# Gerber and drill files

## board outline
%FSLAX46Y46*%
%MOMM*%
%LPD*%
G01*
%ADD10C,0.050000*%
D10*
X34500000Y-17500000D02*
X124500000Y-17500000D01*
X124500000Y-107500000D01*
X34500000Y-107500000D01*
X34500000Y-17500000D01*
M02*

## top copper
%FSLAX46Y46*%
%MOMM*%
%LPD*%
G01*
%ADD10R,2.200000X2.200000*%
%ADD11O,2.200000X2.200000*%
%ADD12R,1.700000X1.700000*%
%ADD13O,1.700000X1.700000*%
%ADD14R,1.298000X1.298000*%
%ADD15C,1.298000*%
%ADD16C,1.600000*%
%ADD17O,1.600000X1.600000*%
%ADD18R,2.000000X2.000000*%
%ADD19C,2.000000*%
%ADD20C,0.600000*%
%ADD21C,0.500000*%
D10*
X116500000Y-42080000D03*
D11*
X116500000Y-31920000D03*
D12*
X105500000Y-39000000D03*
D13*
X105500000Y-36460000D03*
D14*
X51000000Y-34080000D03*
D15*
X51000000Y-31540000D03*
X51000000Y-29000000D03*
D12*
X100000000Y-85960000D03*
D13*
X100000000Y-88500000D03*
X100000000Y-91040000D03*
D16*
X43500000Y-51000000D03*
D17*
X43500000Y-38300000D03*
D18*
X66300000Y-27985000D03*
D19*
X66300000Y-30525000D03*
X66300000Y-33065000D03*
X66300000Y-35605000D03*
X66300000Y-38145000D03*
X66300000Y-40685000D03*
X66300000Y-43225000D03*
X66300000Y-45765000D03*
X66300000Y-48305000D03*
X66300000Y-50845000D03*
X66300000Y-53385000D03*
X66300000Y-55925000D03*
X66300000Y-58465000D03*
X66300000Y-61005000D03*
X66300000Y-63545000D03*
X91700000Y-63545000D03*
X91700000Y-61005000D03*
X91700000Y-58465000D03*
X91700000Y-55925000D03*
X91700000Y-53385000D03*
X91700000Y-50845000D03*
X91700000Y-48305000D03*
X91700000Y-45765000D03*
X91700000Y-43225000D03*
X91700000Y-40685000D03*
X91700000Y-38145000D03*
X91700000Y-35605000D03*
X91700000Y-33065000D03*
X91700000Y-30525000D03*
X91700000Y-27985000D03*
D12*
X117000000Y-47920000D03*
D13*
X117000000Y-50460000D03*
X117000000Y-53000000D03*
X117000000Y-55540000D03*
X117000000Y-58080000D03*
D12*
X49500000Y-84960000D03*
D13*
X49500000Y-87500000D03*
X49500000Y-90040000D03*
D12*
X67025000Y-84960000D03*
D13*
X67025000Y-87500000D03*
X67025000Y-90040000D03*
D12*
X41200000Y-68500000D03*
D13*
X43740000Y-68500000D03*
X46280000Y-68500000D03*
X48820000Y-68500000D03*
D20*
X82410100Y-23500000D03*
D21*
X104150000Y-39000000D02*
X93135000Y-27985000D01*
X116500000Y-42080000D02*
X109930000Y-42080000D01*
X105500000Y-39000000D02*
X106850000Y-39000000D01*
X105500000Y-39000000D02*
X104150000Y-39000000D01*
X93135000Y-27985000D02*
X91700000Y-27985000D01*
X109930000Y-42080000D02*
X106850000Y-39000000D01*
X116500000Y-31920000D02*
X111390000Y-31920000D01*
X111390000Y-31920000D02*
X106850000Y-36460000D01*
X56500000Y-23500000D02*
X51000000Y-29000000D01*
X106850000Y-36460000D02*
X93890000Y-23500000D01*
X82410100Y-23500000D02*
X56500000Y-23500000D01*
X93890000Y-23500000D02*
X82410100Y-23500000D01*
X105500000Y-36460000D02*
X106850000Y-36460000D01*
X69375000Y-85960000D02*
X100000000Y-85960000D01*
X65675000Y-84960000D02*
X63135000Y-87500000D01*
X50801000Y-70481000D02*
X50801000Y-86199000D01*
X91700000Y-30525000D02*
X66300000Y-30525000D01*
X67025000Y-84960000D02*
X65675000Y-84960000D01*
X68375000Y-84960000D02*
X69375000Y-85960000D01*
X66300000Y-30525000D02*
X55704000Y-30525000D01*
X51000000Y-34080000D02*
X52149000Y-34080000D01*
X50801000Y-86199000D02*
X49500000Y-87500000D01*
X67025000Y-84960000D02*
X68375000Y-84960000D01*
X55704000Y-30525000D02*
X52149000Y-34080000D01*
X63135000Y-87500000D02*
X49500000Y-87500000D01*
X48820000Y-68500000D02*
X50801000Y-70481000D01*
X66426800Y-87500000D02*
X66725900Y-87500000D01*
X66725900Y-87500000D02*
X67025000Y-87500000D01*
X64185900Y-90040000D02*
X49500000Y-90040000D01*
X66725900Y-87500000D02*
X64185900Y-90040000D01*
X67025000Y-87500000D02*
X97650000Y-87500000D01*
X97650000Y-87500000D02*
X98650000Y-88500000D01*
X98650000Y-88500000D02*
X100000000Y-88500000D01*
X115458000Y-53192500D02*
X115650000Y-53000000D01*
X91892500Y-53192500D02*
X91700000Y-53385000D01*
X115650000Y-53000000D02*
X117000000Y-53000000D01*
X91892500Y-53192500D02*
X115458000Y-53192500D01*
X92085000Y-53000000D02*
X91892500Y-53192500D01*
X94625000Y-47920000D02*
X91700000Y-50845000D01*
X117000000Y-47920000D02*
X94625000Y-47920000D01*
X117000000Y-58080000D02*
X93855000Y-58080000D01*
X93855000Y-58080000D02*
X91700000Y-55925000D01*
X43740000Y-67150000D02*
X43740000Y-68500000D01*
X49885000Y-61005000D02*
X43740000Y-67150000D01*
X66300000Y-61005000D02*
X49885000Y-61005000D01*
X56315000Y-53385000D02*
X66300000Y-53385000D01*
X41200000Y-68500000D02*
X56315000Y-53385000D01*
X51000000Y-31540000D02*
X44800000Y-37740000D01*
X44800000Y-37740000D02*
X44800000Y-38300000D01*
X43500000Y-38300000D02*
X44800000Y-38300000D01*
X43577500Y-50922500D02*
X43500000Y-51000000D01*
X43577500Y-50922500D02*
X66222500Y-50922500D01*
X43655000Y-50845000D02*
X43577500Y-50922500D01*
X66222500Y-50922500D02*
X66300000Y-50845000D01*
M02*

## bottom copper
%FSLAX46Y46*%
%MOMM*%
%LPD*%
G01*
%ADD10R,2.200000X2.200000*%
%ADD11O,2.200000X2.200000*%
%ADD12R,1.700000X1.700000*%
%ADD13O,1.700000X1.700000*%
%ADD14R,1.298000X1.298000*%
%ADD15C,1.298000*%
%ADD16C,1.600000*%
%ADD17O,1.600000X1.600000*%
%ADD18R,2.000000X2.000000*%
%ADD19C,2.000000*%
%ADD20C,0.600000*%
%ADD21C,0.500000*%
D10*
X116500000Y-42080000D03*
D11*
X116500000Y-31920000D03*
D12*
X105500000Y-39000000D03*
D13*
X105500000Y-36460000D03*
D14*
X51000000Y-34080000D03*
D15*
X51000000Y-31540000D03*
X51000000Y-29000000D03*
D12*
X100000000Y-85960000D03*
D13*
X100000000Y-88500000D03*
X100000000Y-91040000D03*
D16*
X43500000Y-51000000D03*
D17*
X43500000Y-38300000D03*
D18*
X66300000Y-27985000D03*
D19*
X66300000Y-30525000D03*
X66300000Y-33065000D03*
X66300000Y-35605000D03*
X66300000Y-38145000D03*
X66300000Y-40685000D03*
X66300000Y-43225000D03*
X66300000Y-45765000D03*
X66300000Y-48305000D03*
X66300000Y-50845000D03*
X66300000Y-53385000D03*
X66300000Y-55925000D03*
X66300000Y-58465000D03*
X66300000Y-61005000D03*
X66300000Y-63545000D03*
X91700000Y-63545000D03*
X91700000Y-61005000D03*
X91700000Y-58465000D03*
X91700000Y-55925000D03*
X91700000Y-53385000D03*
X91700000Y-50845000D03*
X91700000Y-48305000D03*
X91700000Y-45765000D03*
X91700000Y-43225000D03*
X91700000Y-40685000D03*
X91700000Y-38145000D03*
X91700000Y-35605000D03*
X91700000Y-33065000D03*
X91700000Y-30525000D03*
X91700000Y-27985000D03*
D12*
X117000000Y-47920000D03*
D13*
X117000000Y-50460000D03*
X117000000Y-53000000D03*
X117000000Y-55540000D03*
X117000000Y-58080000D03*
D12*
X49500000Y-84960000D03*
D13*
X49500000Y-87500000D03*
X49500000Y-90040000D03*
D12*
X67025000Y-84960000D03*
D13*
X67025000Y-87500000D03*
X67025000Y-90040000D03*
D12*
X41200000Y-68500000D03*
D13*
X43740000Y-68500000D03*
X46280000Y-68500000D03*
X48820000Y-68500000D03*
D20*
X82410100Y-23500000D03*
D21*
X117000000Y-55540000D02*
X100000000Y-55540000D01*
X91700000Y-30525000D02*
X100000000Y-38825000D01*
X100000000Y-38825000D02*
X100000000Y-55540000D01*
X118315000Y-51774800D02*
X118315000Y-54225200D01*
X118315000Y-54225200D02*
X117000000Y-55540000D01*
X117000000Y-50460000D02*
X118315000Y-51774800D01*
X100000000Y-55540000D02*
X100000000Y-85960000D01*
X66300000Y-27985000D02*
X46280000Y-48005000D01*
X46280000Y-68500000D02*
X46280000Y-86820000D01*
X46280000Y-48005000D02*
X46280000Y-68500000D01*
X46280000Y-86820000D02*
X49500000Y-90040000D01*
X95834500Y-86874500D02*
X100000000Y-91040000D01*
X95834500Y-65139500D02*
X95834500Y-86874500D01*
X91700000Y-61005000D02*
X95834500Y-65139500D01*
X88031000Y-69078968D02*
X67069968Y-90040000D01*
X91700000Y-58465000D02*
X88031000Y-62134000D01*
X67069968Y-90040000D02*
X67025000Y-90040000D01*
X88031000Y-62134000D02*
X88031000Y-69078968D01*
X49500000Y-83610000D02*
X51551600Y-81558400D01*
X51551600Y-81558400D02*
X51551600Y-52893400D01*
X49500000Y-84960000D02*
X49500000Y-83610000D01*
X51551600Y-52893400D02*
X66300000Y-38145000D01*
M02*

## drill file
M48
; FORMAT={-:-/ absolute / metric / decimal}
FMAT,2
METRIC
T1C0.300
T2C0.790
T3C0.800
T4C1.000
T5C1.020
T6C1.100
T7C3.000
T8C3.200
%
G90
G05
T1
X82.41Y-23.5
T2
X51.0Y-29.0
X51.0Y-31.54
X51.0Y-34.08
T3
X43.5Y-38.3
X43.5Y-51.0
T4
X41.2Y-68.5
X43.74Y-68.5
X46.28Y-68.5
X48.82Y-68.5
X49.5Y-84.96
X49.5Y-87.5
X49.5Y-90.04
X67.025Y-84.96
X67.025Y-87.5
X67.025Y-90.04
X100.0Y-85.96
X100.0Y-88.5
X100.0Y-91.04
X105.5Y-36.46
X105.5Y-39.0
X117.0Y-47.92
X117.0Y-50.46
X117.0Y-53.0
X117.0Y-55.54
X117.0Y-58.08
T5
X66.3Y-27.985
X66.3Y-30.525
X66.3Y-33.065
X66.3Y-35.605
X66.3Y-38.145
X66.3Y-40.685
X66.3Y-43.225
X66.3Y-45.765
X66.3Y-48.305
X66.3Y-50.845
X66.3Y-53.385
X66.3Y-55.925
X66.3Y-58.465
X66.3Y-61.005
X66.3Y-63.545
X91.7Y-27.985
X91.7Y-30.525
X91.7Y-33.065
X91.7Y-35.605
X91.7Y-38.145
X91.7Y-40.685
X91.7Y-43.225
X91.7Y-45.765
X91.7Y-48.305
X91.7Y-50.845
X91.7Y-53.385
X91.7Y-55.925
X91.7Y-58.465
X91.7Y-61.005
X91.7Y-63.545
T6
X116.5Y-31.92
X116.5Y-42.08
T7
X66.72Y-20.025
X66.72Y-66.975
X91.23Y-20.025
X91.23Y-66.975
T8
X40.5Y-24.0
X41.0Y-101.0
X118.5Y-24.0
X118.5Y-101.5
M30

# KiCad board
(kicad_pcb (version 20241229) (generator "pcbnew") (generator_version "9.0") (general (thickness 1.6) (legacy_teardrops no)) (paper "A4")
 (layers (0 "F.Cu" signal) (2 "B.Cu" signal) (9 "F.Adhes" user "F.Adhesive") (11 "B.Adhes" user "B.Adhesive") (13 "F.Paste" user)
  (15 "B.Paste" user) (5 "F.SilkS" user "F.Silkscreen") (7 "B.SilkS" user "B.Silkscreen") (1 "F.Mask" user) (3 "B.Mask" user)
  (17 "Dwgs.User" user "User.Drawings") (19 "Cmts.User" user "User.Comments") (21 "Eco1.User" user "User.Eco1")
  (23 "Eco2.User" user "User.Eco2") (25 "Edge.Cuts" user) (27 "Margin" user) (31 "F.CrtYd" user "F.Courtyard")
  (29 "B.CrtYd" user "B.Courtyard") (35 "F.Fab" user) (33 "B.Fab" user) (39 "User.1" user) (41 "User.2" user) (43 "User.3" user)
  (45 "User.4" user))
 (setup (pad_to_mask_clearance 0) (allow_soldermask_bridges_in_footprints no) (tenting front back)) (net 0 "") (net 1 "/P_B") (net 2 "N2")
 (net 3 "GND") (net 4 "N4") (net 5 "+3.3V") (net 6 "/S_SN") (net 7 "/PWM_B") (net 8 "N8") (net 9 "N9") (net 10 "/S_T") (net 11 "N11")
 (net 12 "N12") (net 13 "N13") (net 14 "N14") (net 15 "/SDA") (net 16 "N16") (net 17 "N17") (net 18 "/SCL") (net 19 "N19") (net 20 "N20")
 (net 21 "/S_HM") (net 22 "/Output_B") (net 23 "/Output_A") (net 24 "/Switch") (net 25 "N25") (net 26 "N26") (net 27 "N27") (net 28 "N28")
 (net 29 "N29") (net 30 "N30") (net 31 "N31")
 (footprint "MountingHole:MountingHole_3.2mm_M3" (layer "F.Cu") (at 118.5 101.5)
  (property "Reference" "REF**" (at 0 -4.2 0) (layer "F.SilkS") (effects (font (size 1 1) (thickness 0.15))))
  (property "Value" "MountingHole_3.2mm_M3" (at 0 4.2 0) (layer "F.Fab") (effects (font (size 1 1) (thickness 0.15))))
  (pad "" np_thru_hole circle (at 0 0) (size 3.2 3.2) (drill 3.2) (layers "*.Cu" "*.Mask")))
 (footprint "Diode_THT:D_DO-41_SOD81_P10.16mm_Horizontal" (layer "F.Cu") (at 116.5 42.08 90)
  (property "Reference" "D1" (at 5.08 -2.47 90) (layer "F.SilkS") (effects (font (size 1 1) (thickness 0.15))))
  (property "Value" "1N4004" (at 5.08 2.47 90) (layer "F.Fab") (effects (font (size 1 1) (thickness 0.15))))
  (pad "1" thru_hole rect (at 0 0 90) (size 2.2 2.2) (drill 1.1) (layers "*.Cu" "*.Mask") (remove_unused_layers no) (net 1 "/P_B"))
  (pad "2" thru_hole oval (at 10.16 0 90) (size 2.2 2.2) (drill 1.1) (layers "*.Cu" "*.Mask") (remove_unused_layers no) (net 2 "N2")))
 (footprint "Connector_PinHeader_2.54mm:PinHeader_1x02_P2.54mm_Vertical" (layer "F.Cu") (at 105.5 39 180)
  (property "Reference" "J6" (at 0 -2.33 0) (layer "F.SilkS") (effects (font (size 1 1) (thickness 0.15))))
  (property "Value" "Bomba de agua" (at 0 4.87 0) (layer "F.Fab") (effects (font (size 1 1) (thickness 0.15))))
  (pad "1" thru_hole rect (at 0 0 180) (size 1.7 1.7) (drill 1) (layers "*.Cu" "*.Mask") (remove_unused_layers no) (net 1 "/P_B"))
  (pad "2" thru_hole oval (at 0 2.54 180) (size 1.7 1.7) (drill 1) (layers "*.Cu" "*.Mask") (remove_unused_layers no) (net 2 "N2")))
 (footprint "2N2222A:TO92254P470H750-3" (layer "F.Cu") (at 48.67 31.54 90)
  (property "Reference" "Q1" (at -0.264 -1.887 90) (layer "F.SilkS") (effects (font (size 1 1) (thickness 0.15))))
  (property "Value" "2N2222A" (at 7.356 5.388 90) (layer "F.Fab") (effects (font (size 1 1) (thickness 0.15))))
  (pad "1" thru_hole rect (at -2.54 2.33 90) (size 1.298 1.298) (drill 0.79) (layers "*.Cu" "*.Mask") (remove_unused_layers no)
   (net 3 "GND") (solder_mask_margin 0.102))
  (pad "2" thru_hole circle (at 0 2.33 90) (size 1.298 1.298) (drill 0.79) (layers "*.Cu" "*.Mask") (remove_unused_layers no) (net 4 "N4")
   (solder_mask_margin 0.102))
  (pad "3" thru_hole circle (at 2.54 2.33 90) (size 1.298 1.298) (drill 0.79) (layers "*.Cu" "*.Mask") (remove_unused_layers no)
   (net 2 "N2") (solder_mask_margin 0.102)))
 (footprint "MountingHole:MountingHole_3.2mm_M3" (layer "F.Cu") (at 41 101)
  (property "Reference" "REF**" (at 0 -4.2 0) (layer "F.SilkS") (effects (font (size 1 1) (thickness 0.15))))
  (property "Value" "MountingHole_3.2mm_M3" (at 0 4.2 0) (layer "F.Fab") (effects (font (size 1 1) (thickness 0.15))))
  (pad "" np_thru_hole circle (at 0 0) (size 3.2 3.2) (drill 3.2) (layers "*.Cu" "*.Mask")))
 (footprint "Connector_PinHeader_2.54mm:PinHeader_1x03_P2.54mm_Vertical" (layer "F.Cu") (at 100 85.96)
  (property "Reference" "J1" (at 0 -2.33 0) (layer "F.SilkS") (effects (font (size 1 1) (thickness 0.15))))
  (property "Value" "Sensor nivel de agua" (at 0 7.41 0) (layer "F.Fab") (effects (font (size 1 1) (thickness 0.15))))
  (pad "1" thru_hole rect (at 0 0) (size 1.7 1.7) (drill 1) (layers "*.Cu" "*.Mask") (remove_unused_layers no) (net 3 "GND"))
  (pad "2" thru_hole oval (at 0 2.54) (size 1.7 1.7) (drill 1) (layers "*.Cu" "*.Mask") (remove_unused_layers no) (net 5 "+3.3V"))
  (pad "3" thru_hole oval (at 0 5.08) (size 1.7 1.7) (drill 1) (layers "*.Cu" "*.Mask") (remove_unused_layers no) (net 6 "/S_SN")))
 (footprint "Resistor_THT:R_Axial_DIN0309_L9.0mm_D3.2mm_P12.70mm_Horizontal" (layer "F.Cu") (at 43.5 51 90)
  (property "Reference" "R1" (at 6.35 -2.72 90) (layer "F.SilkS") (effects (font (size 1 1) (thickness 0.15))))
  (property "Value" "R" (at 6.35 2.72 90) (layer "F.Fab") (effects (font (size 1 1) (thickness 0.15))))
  (pad "1" thru_hole circle (at 0 0 90) (size 1.6 1.6) (drill 0.8) (layers "*.Cu" "*.Mask") (remove_unused_layers no) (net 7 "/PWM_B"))
  (pad "2" thru_hole oval (at 12.7 0 90) (size 1.6 1.6) (drill 0.8) (layers "*.Cu" "*.Mask") (remove_unused_layers no) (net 4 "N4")))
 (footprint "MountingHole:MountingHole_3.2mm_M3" (layer "F.Cu") (at 118.5 24)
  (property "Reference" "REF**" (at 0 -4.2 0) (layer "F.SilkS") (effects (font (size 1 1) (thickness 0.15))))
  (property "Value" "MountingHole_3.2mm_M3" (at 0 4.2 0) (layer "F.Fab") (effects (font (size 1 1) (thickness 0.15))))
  (pad "" np_thru_hole circle (at 0 0) (size 3.2 3.2) (drill 3.2) (layers "*.Cu" "*.Mask")))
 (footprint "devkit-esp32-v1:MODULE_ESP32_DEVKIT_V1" (layer "F.Cu") (at 79 43.5)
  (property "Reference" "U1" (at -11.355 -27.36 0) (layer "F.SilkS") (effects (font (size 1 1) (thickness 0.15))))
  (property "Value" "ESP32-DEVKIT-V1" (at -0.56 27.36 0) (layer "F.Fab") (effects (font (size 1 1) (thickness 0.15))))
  (pad "" np_thru_hole circle (at -12.28 -23.475) (size 3 3) (drill 3) (layers "*.Cu" "*.Mask"))
  (pad "" np_thru_hole circle (at -12.28 23.475) (size 3 3) (drill 3) (layers "*.Cu" "*.Mask"))
  (pad "" np_thru_hole circle (at 12.23 -23.475) (size 3 3) (drill 3) (layers "*.Cu" "*.Mask"))
  (pad "" np_thru_hole circle (at 12.23 23.475) (size 3 3) (drill 3) (layers "*.Cu" "*.Mask"))
  (pad "1" thru_hole rect (at -12.7 -15.515) (size 2 2) (drill 1.02) (layers "*.Cu" "*.Mask") (remove_unused_layers no) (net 5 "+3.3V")
   (solder_mask_margin 0.102))
  (pad "2" thru_hole circle (at -12.7 -12.975) (size 2 2) (drill 1.02) (layers "*.Cu" "*.Mask") (remove_unused_layers no) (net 3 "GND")
   (solder_mask_margin 0.102))
  (pad "3" thru_hole circle (at -12.7 -10.435) (size 2 2) (drill 1.02) (layers "*.Cu" "*.Mask") (remove_unused_layers no) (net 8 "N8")
   (solder_mask_margin 0.102))
  (pad "4" thru_hole circle (at -12.7 -7.895) (size 2 2) (drill 1.02) (layers "*.Cu" "*.Mask") (remove_unused_layers no) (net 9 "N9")
   (solder_mask_margin 0.102))
  (pad "5" thru_hole circle (at -12.7 -5.355) (size 2 2) (drill 1.02) (layers "*.Cu" "*.Mask") (remove_unused_layers no) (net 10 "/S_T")
   (solder_mask_margin 0.102))
  (pad "6" thru_hole circle (at -12.7 -2.815) (size 2 2) (drill 1.02) (layers "*.Cu" "*.Mask") (remove_unused_layers no) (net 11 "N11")
   (solder_mask_margin 0.102))
  (pad "7" thru_hole circle (at -12.7 -0.275) (size 2 2) (drill 1.02) (layers "*.Cu" "*.Mask") (remove_unused_layers no) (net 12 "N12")
   (solder_mask_margin 0.102))
  (pad "8" thru_hole circle (at -12.7 2.265) (size 2 2) (drill 1.02) (layers "*.Cu" "*.Mask") (remove_unused_layers no) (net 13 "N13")
   (solder_mask_margin 0.102))
  (pad "9" thru_hole circle (at -12.7 4.805) (size 2 2) (drill 1.02) (layers "*.Cu" "*.Mask") (remove_unused_layers no) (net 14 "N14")
   (solder_mask_margin 0.102))
  (pad "10" thru_hole circle (at -12.7 7.345) (size 2 2) (drill 1.02) (layers "*.Cu" "*.Mask") (remove_unused_layers no) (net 7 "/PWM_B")
   (solder_mask_margin 0.102))
  (pad "11" thru_hole circle (at -12.7 9.885) (size 2 2) (drill 1.02) (layers "*.Cu" "*.Mask") (remove_unused_layers no) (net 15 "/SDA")
   (solder_mask_margin 0.102))
  (pad "12" thru_hole circle (at -12.7 12.425) (size 2 2) (drill 1.02) (layers "*.Cu" "*.Mask") (remove_unused_layers no) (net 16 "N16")
   (solder_mask_margin 0.102))
  (pad "13" thru_hole circle (at -12.7 14.965) (size 2 2) (drill 1.02) (layers "*.Cu" "*.Mask") (remove_unused_layers no) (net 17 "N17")
   (solder_mask_margin 0.102))
  (pad "14" thru_hole circle (at -12.7 17.505) (size 2 2) (drill 1.02) (layers "*.Cu" "*.Mask") (remove_unused_layers no) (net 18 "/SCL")
   (solder_mask_margin 0.102))
  (pad "15" thru_hole circle (at -12.7 20.045) (size 2 2) (drill 1.02) (layers "*.Cu" "*.Mask") (remove_unused_layers no) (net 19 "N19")
   (solder_mask_margin 0.102))
  (pad "16" thru_hole circle (at 12.7 20.045) (size 2 2) (drill 1.02) (layers "*.Cu" "*.Mask") (remove_unused_layers no) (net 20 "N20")
   (solder_mask_margin 0.102))
  (pad "17" thru_hole circle (at 12.7 17.505) (size 2 2) (drill 1.02) (layers "*.Cu" "*.Mask") (remove_unused_layers no) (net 6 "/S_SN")
   (solder_mask_margin 0.102))
  (pad "18" thru_hole circle (at 12.7 14.965) (size 2 2) (drill 1.02) (layers "*.Cu" "*.Mask") (remove_unused_layers no) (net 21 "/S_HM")
   (solder_mask_margin 0.102))
  (pad "19" thru_hole circle (at 12.7 12.425) (size 2 2) (drill 1.02) (layers "*.Cu" "*.Mask") (remove_unused_layers no)
   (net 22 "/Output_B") (solder_mask_margin 0.102))
  (pad "20" thru_hole circle (at 12.7 9.885) (size 2 2) (drill 1.02) (layers "*.Cu" "*.Mask") (remove_unused_layers no) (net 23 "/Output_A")
   (solder_mask_margin 0.102))
  (pad "21" thru_hole circle (at 12.7 7.345) (size 2 2) (drill 1.02) (layers "*.Cu" "*.Mask") (remove_unused_layers no) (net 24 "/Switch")
   (solder_mask_margin 0.102))
  (pad "22" thru_hole circle (at 12.7 4.805) (size 2 2) (drill 1.02) (layers "*.Cu" "*.Mask") (remove_unused_layers no) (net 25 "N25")
   (solder_mask_margin 0.102))
  (pad "23" thru_hole circle (at 12.7 2.265) (size 2 2) (drill 1.02) (layers "*.Cu" "*.Mask") (remove_unused_layers no) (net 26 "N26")
   (solder_mask_margin 0.102))
  (pad "24" thru_hole circle (at 12.7 -0.275) (size 2 2) (drill 1.02) (layers "*.Cu" "*.Mask") (remove_unused_layers no) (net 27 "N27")
   (solder_mask_margin 0.102))
  (pad "25" thru_hole circle (at 12.7 -2.815) (size 2 2) (drill 1.02) (layers "*.Cu" "*.Mask") (remove_unused_layers no) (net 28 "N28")
   (solder_mask_margin 0.102))
  (pad "26" thru_hole circle (at 12.7 -5.355) (size 2 2) (drill 1.02) (layers "*.Cu" "*.Mask") (remove_unused_layers no) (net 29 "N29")
   (solder_mask_margin 0.102))
  (pad "27" thru_hole circle (at 12.7 -7.895) (size 2 2) (drill 1.02) (layers "*.Cu" "*.Mask") (remove_unused_layers no) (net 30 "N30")
   (solder_mask_margin 0.102))
  (pad "28" thru_hole circle (at 12.7 -10.435) (size 2 2) (drill 1.02) (layers "*.Cu" "*.Mask") (remove_unused_layers no) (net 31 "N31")
   (solder_mask_margin 0.102))
  (pad "29" thru_hole circle (at 12.7 -12.975) (size 2 2) (drill 1.02) (layers "*.Cu" "*.Mask") (remove_unused_layers no) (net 3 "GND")
   (solder_mask_margin 0.102))
  (pad "30" thru_hole circle (at 12.7 -15.515) (size 2 2) (drill 1.02) (layers "*.Cu" "*.Mask") (remove_unused_layers no) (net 1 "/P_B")
   (solder_mask_margin 0.102))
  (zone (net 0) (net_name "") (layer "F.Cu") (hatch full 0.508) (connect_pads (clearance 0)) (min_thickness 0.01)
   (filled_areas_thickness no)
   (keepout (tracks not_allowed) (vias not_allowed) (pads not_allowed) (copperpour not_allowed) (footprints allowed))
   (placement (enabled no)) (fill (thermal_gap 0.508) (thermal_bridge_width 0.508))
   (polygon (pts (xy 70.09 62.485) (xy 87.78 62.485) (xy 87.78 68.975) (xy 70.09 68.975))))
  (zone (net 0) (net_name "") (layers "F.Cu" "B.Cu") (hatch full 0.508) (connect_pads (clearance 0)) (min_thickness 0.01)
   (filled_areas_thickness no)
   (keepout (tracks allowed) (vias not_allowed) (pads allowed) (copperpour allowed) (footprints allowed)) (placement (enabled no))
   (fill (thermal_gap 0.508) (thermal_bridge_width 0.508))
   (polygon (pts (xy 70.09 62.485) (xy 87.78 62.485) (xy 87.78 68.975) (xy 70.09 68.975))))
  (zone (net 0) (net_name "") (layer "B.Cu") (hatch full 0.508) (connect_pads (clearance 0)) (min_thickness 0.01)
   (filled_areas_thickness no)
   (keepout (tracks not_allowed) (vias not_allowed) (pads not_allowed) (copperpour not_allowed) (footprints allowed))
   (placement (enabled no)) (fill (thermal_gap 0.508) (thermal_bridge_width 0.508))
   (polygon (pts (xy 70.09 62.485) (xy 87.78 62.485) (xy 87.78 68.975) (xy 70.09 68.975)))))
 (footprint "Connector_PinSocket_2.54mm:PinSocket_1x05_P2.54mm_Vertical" (layer "F.Cu") (at 117 47.92)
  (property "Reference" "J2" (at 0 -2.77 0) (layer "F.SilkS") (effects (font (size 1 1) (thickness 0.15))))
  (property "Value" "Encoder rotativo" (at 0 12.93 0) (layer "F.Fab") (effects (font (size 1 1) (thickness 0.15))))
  (pad "1" thru_hole rect (at 0 0) (size 1.7 1.7) (drill 1) (layers "*.Cu" "*.Mask") (remove_unused_layers no) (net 24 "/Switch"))
  (pad "2" thru_hole oval (at 0 2.54) (size 1.7 1.7) (drill 1) (layers "*.Cu" "*.Mask") (remove_unused_layers no) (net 3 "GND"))
  (pad "3" thru_hole oval (at 0 5.08) (size 1.7 1.7) (drill 1) (layers "*.Cu" "*.Mask") (remove_unused_layers no) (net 23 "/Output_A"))
  (pad "4" thru_hole oval (at 0 7.62) (size 1.7 1.7) (drill 1) (layers "*.Cu" "*.Mask") (remove_unused_layers no) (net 3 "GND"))
  (pad "5" thru_hole oval (at 0 10.16) (size 1.7 1.7) (drill 1) (layers "*.Cu" "*.Mask") (remove_unused_layers no) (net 22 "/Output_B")))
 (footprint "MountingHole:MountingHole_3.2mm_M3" (layer "F.Cu") (at 40.5 24)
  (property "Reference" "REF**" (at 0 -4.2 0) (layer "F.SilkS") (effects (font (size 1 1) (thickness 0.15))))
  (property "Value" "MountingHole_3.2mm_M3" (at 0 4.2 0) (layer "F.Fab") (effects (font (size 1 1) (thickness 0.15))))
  (pad "" np_thru_hole circle (at 0 0) (size 3.2 3.2) (drill 3.2) (layers "*.Cu" "*.Mask")))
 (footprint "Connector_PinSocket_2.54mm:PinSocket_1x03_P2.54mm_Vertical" (layer "F.Cu") (at 49.5 84.96)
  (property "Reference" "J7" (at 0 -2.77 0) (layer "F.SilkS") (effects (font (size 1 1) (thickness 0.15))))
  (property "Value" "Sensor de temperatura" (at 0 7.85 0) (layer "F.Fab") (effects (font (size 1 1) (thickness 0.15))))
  (pad "1" thru_hole rect (at 0 0) (size 1.7 1.7) (drill 1) (layers "*.Cu" "*.Mask") (remove_unused_layers no) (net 10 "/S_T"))
  (pad "2" thru_hole oval (at 0 2.54) (size 1.7 1.7) (drill 1) (layers "*.Cu" "*.Mask") (remove_unused_layers no) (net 3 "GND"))
  (pad "3" thru_hole oval (at 0 5.08) (size 1.7 1.7) (drill 1) (layers "*.Cu" "*.Mask") (remove_unused_layers no) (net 5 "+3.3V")))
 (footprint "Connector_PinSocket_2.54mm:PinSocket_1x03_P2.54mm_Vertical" (layer "F.Cu") (at 67.025 84.96)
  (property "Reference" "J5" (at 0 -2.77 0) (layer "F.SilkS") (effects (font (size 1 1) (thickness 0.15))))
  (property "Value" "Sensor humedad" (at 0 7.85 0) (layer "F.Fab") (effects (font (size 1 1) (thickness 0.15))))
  (pad "1" thru_hole rect (at 0 0) (size 1.7 1.7) (drill 1) (layers "*.Cu" "*.Mask") (remove_unused_layers no) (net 3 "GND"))
  (pad "2" thru_hole oval (at 0 2.54) (size 1.7 1.7) (drill 1) (layers "*.Cu" "*.Mask") (remove_unused_layers no) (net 5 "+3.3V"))
  (pad "3" thru_hole oval (at 0 5.08) (size 1.7 1.7) (drill 1) (layers "*.Cu" "*.Mask") (remove_unused_layers no) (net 21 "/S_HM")))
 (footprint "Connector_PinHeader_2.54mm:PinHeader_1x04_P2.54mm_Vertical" (layer "F.Cu") (at 41.2 68.5 90)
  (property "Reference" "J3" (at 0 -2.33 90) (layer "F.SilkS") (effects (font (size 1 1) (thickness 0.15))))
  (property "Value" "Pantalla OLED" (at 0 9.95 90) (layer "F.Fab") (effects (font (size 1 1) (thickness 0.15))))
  (pad "1" thru_hole rect (at 0 0 90) (size 1.7 1.7) (drill 1) (layers "*.Cu" "*.Mask") (remove_unused_layers no) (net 15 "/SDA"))
  (pad "2" thru_hole oval (at 0 2.54 90) (size 1.7 1.7) (drill 1) (layers "*.Cu" "*.Mask") (remove_unused_layers no) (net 18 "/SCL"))
  (pad "3" thru_hole oval (at 0 5.08 90) (size 1.7 1.7) (drill 1) (layers "*.Cu" "*.Mask") (remove_unused_layers no) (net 5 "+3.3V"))
  (pad "4" thru_hole oval (at 0 7.62 90) (size 1.7 1.7) (drill 1) (layers "*.Cu" "*.Mask") (remove_unused_layers no) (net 3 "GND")))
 (gr_rect (start 34.5 17.5) (end 124.5 107.5) (stroke (width 0.05) (type solid)) (fill no) (layer "Edge.Cuts"))
 (segment (start 104.15 39) (end 93.135 27.985) (width 0.5) (layer "F.Cu") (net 1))
 (segment (start 116.5 42.08) (end 109.93 42.08) (width 0.5) (layer "F.Cu") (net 1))
 (segment (start 105.5 39) (end 106.85 39) (width 0.5) (layer "F.Cu") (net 1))
 (segment (start 105.5 39) (end 104.15 39) (width 0.5) (layer "F.Cu") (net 1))
 (segment (start 93.135 27.985) (end 91.7 27.985) (width 0.5) (layer "F.Cu") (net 1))
 (segment (start 109.93 42.08) (end 106.85 39) (width 0.5) (layer "F.Cu") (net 1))
 (segment (start 116.5 31.92) (end 111.39 31.92) (width 0.5) (layer "F.Cu") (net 2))
 (segment (start 111.39 31.92) (end 106.85 36.46) (width 0.5) (layer "F.Cu") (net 2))
 (segment (start 56.5 23.5) (end 51 29) (width 0.5) (layer "F.Cu") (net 2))
 (segment (start 106.85 36.46) (end 93.89 23.5) (width 0.5) (layer "F.Cu") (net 2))
 (segment (start 82.4101 23.5) (end 56.5 23.5) (width 0.5) (layer "F.Cu") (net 2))
 (segment (start 93.89 23.5) (end 82.4101 23.5) (width 0.5) (layer "F.Cu") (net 2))
 (segment (start 105.5 36.46) (end 106.85 36.46) (width 0.5) (layer "F.Cu") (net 2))
 (via (at 82.4101 23.5) (size 0.6) (drill 0.3) (layers "F.Cu" "B.Cu") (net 2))
 (segment (start 69.375 85.96) (end 100 85.96) (width 0.5) (layer "F.Cu") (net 3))
 (segment (start 65.675 84.96) (end 63.135 87.5) (width 0.5) (layer "F.Cu") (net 3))
 (segment (start 50.801 70.481) (end 50.801 86.199) (width 0.5) (layer "F.Cu") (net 3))
 (segment (start 91.7 30.525) (end 66.3 30.525) (width 0.5) (layer "F.Cu") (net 3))
 (segment (start 67.025 84.96) (end 65.675 84.96) (width 0.5) (layer "F.Cu") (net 3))
 (segment (start 68.375 84.96) (end 69.375 85.96) (width 0.5) (layer "F.Cu") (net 3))
 (segment (start 66.3 30.525) (end 55.704 30.525) (width 0.5) (layer "F.Cu") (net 3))
 (segment (start 51 34.08) (end 52.149 34.08) (width 0.5) (layer "F.Cu") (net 3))
 (segment (start 50.801 86.199) (end 49.5 87.5) (width 0.5) (layer "F.Cu") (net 3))
 (segment (start 67.025 84.96) (end 68.375 84.96) (width 0.5) (layer "F.Cu") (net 3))
 (segment (start 55.704 30.525) (end 52.149 34.08) (width 0.5) (layer "F.Cu") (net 3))
 (segment (start 63.135 87.5) (end 49.5 87.5) (width 0.5) (layer "F.Cu") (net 3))
 (segment (start 48.82 68.5) (end 50.801 70.481) (width 0.5) (layer "F.Cu") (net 3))
 (segment (start 117 55.54) (end 100 55.54) (width 0.5) (layer "B.Cu") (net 3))
 (segment (start 91.7 30.525) (end 100 38.825) (width 0.5) (layer "B.Cu") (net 3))
 (segment (start 100 38.825) (end 100 55.54) (width 0.5) (layer "B.Cu") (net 3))
 (segment (start 118.315 51.7748) (end 118.315 54.2252) (width 0.5) (layer "B.Cu") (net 3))
 (segment (start 118.315 54.2252) (end 117 55.54) (width 0.5) (layer "B.Cu") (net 3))
 (segment (start 117 50.46) (end 118.315 51.7748) (width 0.5) (layer "B.Cu") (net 3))
 (segment (start 100 55.54) (end 100 85.96) (width 0.5) (layer "B.Cu") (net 3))
 (segment (start 66.4268 87.5) (end 66.7259 87.5) (width 0.5) (layer "F.Cu") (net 5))
 (segment (start 66.7259 87.5) (end 67.025 87.5) (width 0.5) (layer "F.Cu") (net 5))
 (segment (start 64.1859 90.04) (end 49.5 90.04) (width 0.5) (layer "F.Cu") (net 5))
 (segment (start 66.7259 87.5) (end 64.1859 90.04) (width 0.5) (layer "F.Cu") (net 5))
 (segment (start 67.025 87.5) (end 97.65 87.5) (width 0.5) (layer "F.Cu") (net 5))
 (segment (start 97.65 87.5) (end 98.65 88.5) (width 0.5) (layer "F.Cu") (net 5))
 (segment (start 98.65 88.5) (end 100 88.5) (width 0.5) (layer "F.Cu") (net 5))
 (segment (start 66.3 27.985) (end 46.28 48.005) (width 0.5) (layer "B.Cu") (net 5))
 (segment (start 46.28 68.5) (end 46.28 86.82) (width 0.5) (layer "B.Cu") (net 5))
 (segment (start 46.28 48.005) (end 46.28 68.5) (width 0.5) (layer "B.Cu") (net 5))
 (segment (start 46.28 86.82) (end 49.5 90.04) (width 0.5) (layer "B.Cu") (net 5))
 (segment (start 95.8345 86.8745) (end 100 91.04) (width 0.5) (layer "B.Cu") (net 6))
 (segment (start 95.8345 65.1395) (end 95.8345 86.8745) (width 0.5) (layer "B.Cu") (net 6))
 (segment (start 91.7 61.005) (end 95.8345 65.1395) (width 0.5) (layer "B.Cu") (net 6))
 (segment (start 115.458 53.1925) (end 115.65 53) (width 0.5) (layer "F.Cu") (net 23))
 (segment (start 91.8925 53.1925) (end 91.7 53.385) (width 0.5) (layer "F.Cu") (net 23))
 (segment (start 115.65 53) (end 117 53) (width 0.5) (layer "F.Cu") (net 23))
 (segment (start 91.8925 53.1925) (end 115.458 53.1925) (width 0.5) (layer "F.Cu") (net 23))
 (segment (start 92.085 53) (end 91.8925 53.1925) (width 0.5) (layer "F.Cu") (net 23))
 (segment (start 94.625 47.92) (end 91.7 50.845) (width 0.5) (layer "F.Cu") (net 24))
 (segment (start 117 47.92) (end 94.625 47.92) (width 0.5) (layer "F.Cu") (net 24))
 (segment (start 117 58.08) (end 93.855 58.08) (width 0.5) (layer "F.Cu") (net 22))
 (segment (start 93.855 58.08) (end 91.7 55.925) (width 0.5) (layer "F.Cu") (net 22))
 (segment (start 43.74 67.15) (end 43.74 68.5) (width 0.5) (layer "F.Cu") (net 18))
 (segment (start 49.885 61.005) (end 43.74 67.15) (width 0.5) (layer "F.Cu") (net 18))
 (segment (start 66.3 61.005) (end 49.885 61.005) (width 0.5) (layer "F.Cu") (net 18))
 (segment (start 56.315 53.385) (end 66.3 53.385) (width 0.5) (layer "F.Cu") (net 15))
 (segment (start 41.2 68.5) (end 56.315 53.385) (width 0.5) (layer "F.Cu") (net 15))
 (segment (start 88.031 69.078968) (end 67.069968 90.04) (width 0.5) (layer "B.Cu") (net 21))
 (segment (start 91.7 58.465) (end 88.031 62.134) (width 0.5) (layer "B.Cu") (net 21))
 (segment (start 67.069968 90.04) (end 67.025 90.04) (width 0.5) (layer "B.Cu") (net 21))
 (segment (start 88.031 62.134) (end 88.031 69.078968) (width 0.5) (layer "B.Cu") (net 21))
 (segment (start 49.5 83.61) (end 51.5516 81.5584) (width 0.5) (layer "B.Cu") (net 10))
 (segment (start 51.5516 81.5584) (end 51.5516 52.8934) (width 0.5) (layer "B.Cu") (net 10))
 (segment (start 49.5 84.96) (end 49.5 83.61) (width 0.5) (layer "B.Cu") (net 10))
 (segment (start 51.5516 52.8934) (end 66.3 38.145) (width 0.5) (layer "B.Cu") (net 10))
 (segment (start 51 31.54) (end 44.8 37.74) (width 0.5) (layer "F.Cu") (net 4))
 (segment (start 44.8 37.74) (end 44.8 38.3) (width 0.5) (layer "F.Cu") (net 4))
 (segment (start 43.5 38.3) (end 44.8 38.3) (width 0.5) (layer "F.Cu") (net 4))
 (segment (start 43.5775 50.9225) (end 43.5 51) (width 0.5) (layer "F.Cu") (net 7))
 (segment (start 43.5775 50.9225) (end 66.2225 50.9225) (width 0.5) (layer "F.Cu") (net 7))
 (segment (start 43.655 50.845) (end 43.5775 50.9225) (width 0.5) (layer "F.Cu") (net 7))
 (segment (start 66.2225 50.9225) (end 66.3 50.845) (width 0.5) (layer "F.Cu") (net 7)))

